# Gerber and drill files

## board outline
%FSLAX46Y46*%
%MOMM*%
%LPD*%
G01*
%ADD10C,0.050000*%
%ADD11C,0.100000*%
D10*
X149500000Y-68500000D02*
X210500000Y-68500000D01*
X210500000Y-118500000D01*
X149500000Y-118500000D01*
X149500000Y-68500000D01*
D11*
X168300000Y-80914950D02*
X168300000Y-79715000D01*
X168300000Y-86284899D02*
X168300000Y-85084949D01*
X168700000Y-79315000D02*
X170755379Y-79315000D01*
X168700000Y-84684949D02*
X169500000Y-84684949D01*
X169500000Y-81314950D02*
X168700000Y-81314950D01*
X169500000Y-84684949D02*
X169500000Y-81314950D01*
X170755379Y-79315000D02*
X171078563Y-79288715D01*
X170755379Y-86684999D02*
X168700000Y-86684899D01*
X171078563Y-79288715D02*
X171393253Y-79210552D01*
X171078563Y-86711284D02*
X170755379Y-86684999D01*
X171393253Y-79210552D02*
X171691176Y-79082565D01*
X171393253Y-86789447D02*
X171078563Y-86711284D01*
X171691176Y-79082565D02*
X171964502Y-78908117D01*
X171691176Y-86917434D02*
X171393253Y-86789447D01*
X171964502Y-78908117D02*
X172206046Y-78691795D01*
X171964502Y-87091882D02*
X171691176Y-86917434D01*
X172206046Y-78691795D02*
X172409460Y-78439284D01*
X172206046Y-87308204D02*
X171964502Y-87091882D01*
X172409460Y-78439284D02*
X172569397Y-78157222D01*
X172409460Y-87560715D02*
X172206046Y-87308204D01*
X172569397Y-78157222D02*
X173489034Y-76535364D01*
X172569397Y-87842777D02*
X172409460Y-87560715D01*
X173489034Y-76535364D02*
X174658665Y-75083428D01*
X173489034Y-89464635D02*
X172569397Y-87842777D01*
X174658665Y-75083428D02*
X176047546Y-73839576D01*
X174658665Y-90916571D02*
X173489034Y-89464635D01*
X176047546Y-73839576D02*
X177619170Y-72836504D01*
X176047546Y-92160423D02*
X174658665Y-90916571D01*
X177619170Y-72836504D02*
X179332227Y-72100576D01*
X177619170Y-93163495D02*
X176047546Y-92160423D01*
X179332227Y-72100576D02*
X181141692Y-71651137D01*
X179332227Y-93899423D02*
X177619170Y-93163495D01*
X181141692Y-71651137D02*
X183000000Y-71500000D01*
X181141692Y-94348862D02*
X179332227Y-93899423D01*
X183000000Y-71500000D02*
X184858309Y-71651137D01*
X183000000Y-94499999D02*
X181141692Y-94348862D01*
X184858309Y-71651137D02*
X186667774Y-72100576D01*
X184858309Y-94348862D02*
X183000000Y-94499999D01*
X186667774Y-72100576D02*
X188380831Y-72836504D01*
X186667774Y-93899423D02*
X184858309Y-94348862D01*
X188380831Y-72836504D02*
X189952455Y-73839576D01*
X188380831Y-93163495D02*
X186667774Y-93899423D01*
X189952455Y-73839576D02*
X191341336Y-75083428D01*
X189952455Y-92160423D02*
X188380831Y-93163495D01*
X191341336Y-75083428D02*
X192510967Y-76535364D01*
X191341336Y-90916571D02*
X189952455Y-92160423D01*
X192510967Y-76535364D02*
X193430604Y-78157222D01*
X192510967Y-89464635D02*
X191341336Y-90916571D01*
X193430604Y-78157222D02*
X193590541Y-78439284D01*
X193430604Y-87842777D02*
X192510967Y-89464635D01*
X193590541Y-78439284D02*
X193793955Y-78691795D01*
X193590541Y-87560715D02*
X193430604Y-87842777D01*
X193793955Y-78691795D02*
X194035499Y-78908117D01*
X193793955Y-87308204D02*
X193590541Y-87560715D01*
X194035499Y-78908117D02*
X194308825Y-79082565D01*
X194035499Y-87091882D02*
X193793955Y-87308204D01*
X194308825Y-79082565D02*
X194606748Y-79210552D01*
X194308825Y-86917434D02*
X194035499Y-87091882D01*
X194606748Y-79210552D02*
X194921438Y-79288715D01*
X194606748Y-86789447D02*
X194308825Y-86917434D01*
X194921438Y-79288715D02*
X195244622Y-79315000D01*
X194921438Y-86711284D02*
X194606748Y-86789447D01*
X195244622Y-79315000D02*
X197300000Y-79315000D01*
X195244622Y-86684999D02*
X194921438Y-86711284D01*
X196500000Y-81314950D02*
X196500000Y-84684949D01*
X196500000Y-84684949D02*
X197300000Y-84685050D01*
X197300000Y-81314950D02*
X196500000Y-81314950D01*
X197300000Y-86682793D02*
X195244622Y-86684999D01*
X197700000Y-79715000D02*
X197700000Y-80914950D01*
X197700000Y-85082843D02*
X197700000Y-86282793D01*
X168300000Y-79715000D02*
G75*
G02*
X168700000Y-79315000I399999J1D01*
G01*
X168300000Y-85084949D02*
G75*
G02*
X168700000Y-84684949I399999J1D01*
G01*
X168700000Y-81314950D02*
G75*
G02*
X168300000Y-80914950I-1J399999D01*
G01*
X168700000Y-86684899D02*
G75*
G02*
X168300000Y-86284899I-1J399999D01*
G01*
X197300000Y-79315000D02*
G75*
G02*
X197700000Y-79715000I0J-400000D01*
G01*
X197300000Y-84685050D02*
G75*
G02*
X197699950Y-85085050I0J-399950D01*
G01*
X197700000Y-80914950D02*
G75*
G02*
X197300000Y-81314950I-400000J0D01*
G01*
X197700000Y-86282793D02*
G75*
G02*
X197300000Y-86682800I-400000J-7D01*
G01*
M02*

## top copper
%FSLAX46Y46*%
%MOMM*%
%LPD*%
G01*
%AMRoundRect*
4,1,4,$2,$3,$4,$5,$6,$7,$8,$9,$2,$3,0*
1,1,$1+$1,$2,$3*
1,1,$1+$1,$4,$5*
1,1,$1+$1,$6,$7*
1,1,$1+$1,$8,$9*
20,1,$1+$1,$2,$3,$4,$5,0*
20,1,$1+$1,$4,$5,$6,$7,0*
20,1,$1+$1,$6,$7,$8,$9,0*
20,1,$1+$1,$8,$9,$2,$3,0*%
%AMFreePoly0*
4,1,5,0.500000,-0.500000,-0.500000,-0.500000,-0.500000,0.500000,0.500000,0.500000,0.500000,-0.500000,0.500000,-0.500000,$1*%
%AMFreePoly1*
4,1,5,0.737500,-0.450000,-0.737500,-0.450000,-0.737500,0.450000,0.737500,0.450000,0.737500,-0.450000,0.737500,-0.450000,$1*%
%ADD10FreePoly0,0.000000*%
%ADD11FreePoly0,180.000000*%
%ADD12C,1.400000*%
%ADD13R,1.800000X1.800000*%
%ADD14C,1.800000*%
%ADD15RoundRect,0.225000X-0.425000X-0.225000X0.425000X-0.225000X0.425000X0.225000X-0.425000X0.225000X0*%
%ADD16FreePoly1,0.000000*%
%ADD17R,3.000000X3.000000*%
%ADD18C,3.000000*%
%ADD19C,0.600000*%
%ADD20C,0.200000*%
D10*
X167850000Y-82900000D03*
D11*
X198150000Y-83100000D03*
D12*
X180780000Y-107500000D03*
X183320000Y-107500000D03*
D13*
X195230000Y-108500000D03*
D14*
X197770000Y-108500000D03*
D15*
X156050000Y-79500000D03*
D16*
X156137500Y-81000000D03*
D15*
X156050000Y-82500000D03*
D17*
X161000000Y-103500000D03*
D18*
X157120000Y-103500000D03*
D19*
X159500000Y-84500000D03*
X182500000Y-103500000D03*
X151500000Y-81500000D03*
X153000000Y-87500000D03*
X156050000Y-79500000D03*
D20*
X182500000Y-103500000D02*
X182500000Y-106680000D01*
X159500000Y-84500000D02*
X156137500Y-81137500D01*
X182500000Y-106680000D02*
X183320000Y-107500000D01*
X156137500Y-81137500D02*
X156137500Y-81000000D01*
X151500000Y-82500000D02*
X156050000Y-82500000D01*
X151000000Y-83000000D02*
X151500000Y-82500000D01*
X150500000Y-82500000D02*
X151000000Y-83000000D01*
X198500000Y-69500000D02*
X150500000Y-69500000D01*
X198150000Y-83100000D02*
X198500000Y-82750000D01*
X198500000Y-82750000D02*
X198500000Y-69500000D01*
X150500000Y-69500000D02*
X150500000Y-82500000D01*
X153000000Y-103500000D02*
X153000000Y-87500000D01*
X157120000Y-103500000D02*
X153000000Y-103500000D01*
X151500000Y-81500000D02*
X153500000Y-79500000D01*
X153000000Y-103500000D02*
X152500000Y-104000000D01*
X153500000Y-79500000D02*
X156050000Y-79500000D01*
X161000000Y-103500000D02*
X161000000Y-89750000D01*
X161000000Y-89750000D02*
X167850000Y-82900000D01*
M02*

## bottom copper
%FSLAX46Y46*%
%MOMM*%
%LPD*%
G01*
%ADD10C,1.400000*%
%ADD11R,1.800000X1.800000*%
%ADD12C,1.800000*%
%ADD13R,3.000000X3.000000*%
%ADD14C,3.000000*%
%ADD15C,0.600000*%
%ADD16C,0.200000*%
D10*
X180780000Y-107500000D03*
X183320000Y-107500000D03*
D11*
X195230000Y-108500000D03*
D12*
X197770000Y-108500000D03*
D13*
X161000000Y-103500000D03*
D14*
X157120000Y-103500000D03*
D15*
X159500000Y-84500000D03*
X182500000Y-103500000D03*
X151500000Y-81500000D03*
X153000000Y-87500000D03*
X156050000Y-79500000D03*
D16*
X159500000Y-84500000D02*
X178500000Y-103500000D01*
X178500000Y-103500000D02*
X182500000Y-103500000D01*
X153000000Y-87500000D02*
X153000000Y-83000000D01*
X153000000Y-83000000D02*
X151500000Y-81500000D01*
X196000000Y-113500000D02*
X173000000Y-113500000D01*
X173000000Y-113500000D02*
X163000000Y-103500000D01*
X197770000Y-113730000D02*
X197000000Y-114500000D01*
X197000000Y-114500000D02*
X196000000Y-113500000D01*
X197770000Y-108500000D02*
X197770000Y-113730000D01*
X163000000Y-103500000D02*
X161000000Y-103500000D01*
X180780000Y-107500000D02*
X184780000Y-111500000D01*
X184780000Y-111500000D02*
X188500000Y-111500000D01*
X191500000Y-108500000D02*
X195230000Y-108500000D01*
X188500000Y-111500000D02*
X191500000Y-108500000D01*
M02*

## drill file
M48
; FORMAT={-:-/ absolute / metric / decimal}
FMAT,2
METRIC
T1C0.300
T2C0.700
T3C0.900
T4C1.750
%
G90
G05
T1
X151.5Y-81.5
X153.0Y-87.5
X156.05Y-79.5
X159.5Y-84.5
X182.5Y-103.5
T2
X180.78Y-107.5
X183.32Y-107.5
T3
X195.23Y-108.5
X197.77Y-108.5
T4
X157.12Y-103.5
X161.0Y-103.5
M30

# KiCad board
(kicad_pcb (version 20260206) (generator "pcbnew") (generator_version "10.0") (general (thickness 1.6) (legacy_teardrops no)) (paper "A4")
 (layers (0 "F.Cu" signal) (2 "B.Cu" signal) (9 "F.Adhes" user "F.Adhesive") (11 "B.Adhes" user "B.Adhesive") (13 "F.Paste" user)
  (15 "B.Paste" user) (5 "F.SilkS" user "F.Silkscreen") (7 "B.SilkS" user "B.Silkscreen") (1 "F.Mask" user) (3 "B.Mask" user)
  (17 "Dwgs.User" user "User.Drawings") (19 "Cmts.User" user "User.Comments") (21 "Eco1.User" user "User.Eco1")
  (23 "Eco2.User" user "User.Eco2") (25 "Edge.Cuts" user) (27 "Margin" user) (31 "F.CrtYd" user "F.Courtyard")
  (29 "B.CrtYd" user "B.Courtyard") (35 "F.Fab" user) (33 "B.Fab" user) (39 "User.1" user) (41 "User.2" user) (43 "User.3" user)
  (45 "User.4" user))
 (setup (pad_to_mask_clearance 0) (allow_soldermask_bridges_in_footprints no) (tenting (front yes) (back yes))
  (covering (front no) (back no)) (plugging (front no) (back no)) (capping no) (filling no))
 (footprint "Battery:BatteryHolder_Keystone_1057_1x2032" (layer "F.Cu") (at 183 83)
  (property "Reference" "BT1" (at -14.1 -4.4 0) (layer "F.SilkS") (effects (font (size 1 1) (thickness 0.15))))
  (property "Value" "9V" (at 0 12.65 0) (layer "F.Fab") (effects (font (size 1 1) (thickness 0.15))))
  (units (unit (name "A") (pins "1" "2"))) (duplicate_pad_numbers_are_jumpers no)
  (fp_line (start -14.7 -2.08505) (end -14.7 -3.285) (stroke (width 0.1) (type solid)) (layer "Edge.Cuts"))
  (fp_line (start -14.7 3.284899) (end -14.7 2.084949) (stroke (width 0.1) (type solid)) (layer "Edge.Cuts"))
  (fp_line (start -14.3 -3.685) (end -12.244621 -3.685) (stroke (width 0.1) (type solid)) (layer "Edge.Cuts"))
  (fp_line (start -14.3 1.684949) (end -13.5 1.684949) (stroke (width 0.1) (type solid)) (layer "Edge.Cuts"))
  (fp_line (start -13.5 -1.68505) (end -14.3 -1.68505) (stroke (width 0.1) (type solid)) (layer "Edge.Cuts"))
  (fp_line (start -13.5 1.684949) (end -13.5 -1.68505) (stroke (width 0.1) (type solid)) (layer "Edge.Cuts"))
  (fp_line (start -12.244621 -3.685) (end -11.921437 -3.711285) (stroke (width 0.1) (type solid)) (layer "Edge.Cuts"))
  (fp_line (start -12.244621 3.684999) (end -14.3 3.684899) (stroke (width 0.1) (type solid)) (layer "Edge.Cuts"))
  (fp_line (start -11.921437 -3.711285) (end -11.606747 -3.789448) (stroke (width 0.1) (type solid)) (layer "Edge.Cuts"))
  (fp_line (start -11.921437 3.711284) (end -12.244621 3.684999) (stroke (width 0.1) (type solid)) (layer "Edge.Cuts"))
  (fp_line (start -11.606747 -3.789448) (end -11.308824 -3.917435) (stroke (width 0.1) (type solid)) (layer "Edge.Cuts"))
  (fp_line (start -11.606747 3.789447) (end -11.921437 3.711284) (stroke (width 0.1) (type solid)) (layer "Edge.Cuts"))
  (fp_line (start -11.308824 -3.917435) (end -11.035498 -4.091883) (stroke (width 0.1) (type solid)) (layer "Edge.Cuts"))
  (fp_line (start -11.308824 3.917434) (end -11.606747 3.789447) (stroke (width 0.1) (type solid)) (layer "Edge.Cuts"))
  (fp_line (start -11.035498 -4.091883) (end -10.793954 -4.308205) (stroke (width 0.1) (type solid)) (layer "Edge.Cuts"))
  (fp_line (start -11.035498 4.091882) (end -11.308824 3.917434) (stroke (width 0.1) (type solid)) (layer "Edge.Cuts"))
  (fp_line (start -10.793954 -4.308205) (end -10.59054 -4.560716) (stroke (width 0.1) (type solid)) (layer "Edge.Cuts"))
  (fp_line (start -10.793954 4.308204) (end -11.035498 4.091882) (stroke (width 0.1) (type solid)) (layer "Edge.Cuts"))
  (fp_line (start -10.59054 -4.560716) (end -10.430603 -4.842778) (stroke (width 0.1) (type solid)) (layer "Edge.Cuts"))
  (fp_line (start -10.59054 4.560715) (end -10.793954 4.308204) (stroke (width 0.1) (type solid)) (layer "Edge.Cuts"))
  (fp_line (start -10.430603 -4.842778) (end -9.510966 -6.464636) (stroke (width 0.1) (type solid)) (layer "Edge.Cuts"))
  (fp_line (start -10.430603 4.842777) (end -10.59054 4.560715) (stroke (width 0.1) (type solid)) (layer "Edge.Cuts"))
  (fp_line (start -9.510966 -6.464636) (end -8.341335 -7.916572) (stroke (width 0.1) (type solid)) (layer "Edge.Cuts"))
  (fp_line (start -9.510966 6.464635) (end -10.430603 4.842777) (stroke (width 0.1) (type solid)) (layer "Edge.Cuts"))
  (fp_line (start -8.341335 -7.916572) (end -6.952454 -9.160424) (stroke (width 0.1) (type solid)) (layer "Edge.Cuts"))
  (fp_line (start -8.341335 7.916571) (end -9.510966 6.464635) (stroke (width 0.1) (type solid)) (layer "Edge.Cuts"))
  (fp_line (start -6.952454 -9.160424) (end -5.38083 -10.163496) (stroke (width 0.1) (type solid)) (layer "Edge.Cuts"))
  (fp_line (start -6.952454 9.160423) (end -8.341335 7.916571) (stroke (width 0.1) (type solid)) (layer "Edge.Cuts"))
  (fp_line (start -5.38083 -10.163496) (end -3.667773 -10.899424) (stroke (width 0.1) (type solid)) (layer "Edge.Cuts"))
  (fp_line (start -5.38083 10.163495) (end -6.952454 9.160423) (stroke (width 0.1) (type solid)) (layer "Edge.Cuts"))
  (fp_line (start -3.667773 -10.899424) (end -1.858308 -11.348863) (stroke (width 0.1) (type solid)) (layer "Edge.Cuts"))
  (fp_line (start -3.667773 10.899423) (end -5.38083 10.163495) (stroke (width 0.1) (type solid)) (layer "Edge.Cuts"))
  (fp_line (start -1.858308 -11.348863) (end 0 -11.5) (stroke (width 0.1) (type solid)) (layer "Edge.Cuts"))
  (fp_line (start -1.858308 11.348862) (end -3.667773 10.899423) (stroke (width 0.1) (type solid)) (layer "Edge.Cuts"))
  (fp_line (start 0 -11.5) (end 1.858309 -11.348863) (stroke (width 0.1) (type solid)) (layer "Edge.Cuts"))
  (fp_line (start 0 11.499999) (end -1.858308 11.348862) (stroke (width 0.1) (type solid)) (layer "Edge.Cuts"))
  (fp_line (start 1.858309 -11.348863) (end 3.667774 -10.899424) (stroke (width 0.1) (type solid)) (layer "Edge.Cuts"))
  (fp_line (start 1.858309 11.348862) (end 0 11.499999) (stroke (width 0.1) (type solid)) (layer "Edge.Cuts"))
  (fp_line (start 3.667774 -10.899424) (end 5.380831 -10.163496) (stroke (width 0.1) (type solid)) (layer "Edge.Cuts"))
  (fp_line (start 3.667774 10.899423) (end 1.858309 11.348862) (stroke (width 0.1) (type solid)) (layer "Edge.Cuts"))
  (fp_line (start 5.380831 -10.163496) (end 6.952455 -9.160424) (stroke (width 0.1) (type solid)) (layer "Edge.Cuts"))
  (fp_line (start 5.380831 10.163495) (end 3.667774 10.899423) (stroke (width 0.1) (type solid)) (layer "Edge.Cuts"))
  (fp_line (start 6.952455 -9.160424) (end 8.341336 -7.916572) (stroke (width 0.1) (type solid)) (layer "Edge.Cuts"))
  (fp_line (start 6.952455 9.160423) (end 5.380831 10.163495) (stroke (width 0.1) (type solid)) (layer "Edge.Cuts"))
  (fp_line (start 8.341336 -7.916572) (end 9.510967 -6.464636) (stroke (width 0.1) (type solid)) (layer "Edge.Cuts"))
  (fp_line (start 8.341336 7.916571) (end 6.952455 9.160423) (stroke (width 0.1) (type solid)) (layer "Edge.Cuts"))
  (fp_line (start 9.510967 -6.464636) (end 10.430604 -4.842778) (stroke (width 0.1) (type solid)) (layer "Edge.Cuts"))
  (fp_line (start 9.510967 6.464635) (end 8.341336 7.916571) (stroke (width 0.1) (type solid)) (layer "Edge.Cuts"))
  (fp_line (start 10.430604 -4.842778) (end 10.590541 -4.560716) (stroke (width 0.1) (type solid)) (layer "Edge.Cuts"))
  (fp_line (start 10.430604 4.842777) (end 9.510967 6.464635) (stroke (width 0.1) (type solid)) (layer "Edge.Cuts"))
  (fp_line (start 10.590541 -4.560716) (end 10.793955 -4.308205) (stroke (width 0.1) (type solid)) (layer "Edge.Cuts"))
  (fp_line (start 10.590541 4.560715) (end 10.430604 4.842777) (stroke (width 0.1) (type solid)) (layer "Edge.Cuts"))
  (fp_line (start 10.793955 -4.308205) (end 11.035499 -4.091883) (stroke (width 0.1) (type solid)) (layer "Edge.Cuts"))
  (fp_line (start 10.793955 4.308204) (end 10.590541 4.560715) (stroke (width 0.1) (type solid)) (layer "Edge.Cuts"))
  (fp_line (start 11.035499 -4.091883) (end 11.308825 -3.917435) (stroke (width 0.1) (type solid)) (layer "Edge.Cuts"))
  (fp_line (start 11.035499 4.091882) (end 10.793955 4.308204) (stroke (width 0.1) (type solid)) (layer "Edge.Cuts"))
  (fp_line (start 11.308825 -3.917435) (end 11.606748 -3.789448) (stroke (width 0.1) (type solid)) (layer "Edge.Cuts"))
  (fp_line (start 11.308825 3.917434) (end 11.035499 4.091882) (stroke (width 0.1) (type solid)) (layer "Edge.Cuts"))
  (fp_line (start 11.606748 -3.789448) (end 11.921438 -3.711285) (stroke (width 0.1) (type solid)) (layer "Edge.Cuts"))
  (fp_line (start 11.606748 3.789447) (end 11.308825 3.917434) (stroke (width 0.1) (type solid)) (layer "Edge.Cuts"))
  (fp_line (start 11.921438 -3.711285) (end 12.244622 -3.685) (stroke (width 0.1) (type solid)) (layer "Edge.Cuts"))
  (fp_line (start 11.921438 3.711284) (end 11.606748 3.789447) (stroke (width 0.1) (type solid)) (layer "Edge.Cuts"))
  (fp_line (start 12.244622 -3.685) (end 14.3 -3.685) (stroke (width 0.1) (type solid)) (layer "Edge.Cuts"))
  (fp_line (start 12.244622 3.684999) (end 11.921438 3.711284) (stroke (width 0.1) (type solid)) (layer "Edge.Cuts"))
  (fp_line (start 13.5 -1.68505) (end 13.5 1.684949) (stroke (width 0.1) (type solid)) (layer "Edge.Cuts"))
  (fp_line (start 13.5 1.684949) (end 14.3 1.68505) (stroke (width 0.1) (type solid)) (layer "Edge.Cuts"))
  (fp_line (start 14.3 -1.68505) (end 13.5 -1.68505) (stroke (width 0.1) (type solid)) (layer "Edge.Cuts"))
  (fp_line (start 14.3 3.682793) (end 12.244622 3.684999) (stroke (width 0.1) (type solid)) (layer "Edge.Cuts"))
  (fp_line (start 14.7 -3.285) (end 14.7 -2.08505) (stroke (width 0.1) (type solid)) (layer "Edge.Cuts"))
  (fp_line (start 14.7 2.082843) (end 14.7 3.282793) (stroke (width 0.1) (type solid)) (layer "Edge.Cuts"))
  (fp_arc (start -14.7 -3.285) (mid -14.582843 -3.567843) (end -14.3 -3.685) (stroke (width 0.1) (type solid)) (layer "Edge.Cuts"))
  (fp_arc (start -14.7 2.084949) (mid -14.582843 1.802106) (end -14.3 1.684949) (stroke (width 0.1) (type solid)) (layer "Edge.Cuts"))
  (fp_arc (start -14.3 -1.68505) (mid -14.582843 -1.802207) (end -14.7 -2.08505) (stroke (width 0.1) (type solid)) (layer "Edge.Cuts"))
  (fp_arc (start -14.3 3.684899) (mid -14.582843 3.567742) (end -14.7 3.284899) (stroke (width 0.1) (type solid)) (layer "Edge.Cuts"))
  (fp_arc (start 14.3 -3.685) (mid 14.582843 -3.567843) (end 14.7 -3.285) (stroke (width 0.1) (type solid)) (layer "Edge.Cuts"))
  (fp_arc (start 14.3 1.68505) (mid 14.582843 1.802207) (end 14.7 2.08505) (stroke (width 0.1) (type solid)) (layer "Edge.Cuts"))
  (fp_arc (start 14.7 -2.08505) (mid 14.582843 -1.802207) (end 14.3 -1.68505) (stroke (width 0.1) (type solid)) (layer "Edge.Cuts"))
  (fp_arc (start 14.7 3.282793) (mid 14.582843 3.565636) (end 14.3 3.682793) (stroke (width 0.1) (type solid)) (layer "Edge.Cuts"))
  (pad "1" smd custom (at -15.15 -0.1) (size 1 1) (layers "F.Cu" "F.Mask" "F.Paste") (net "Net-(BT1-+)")
   (options (clearance outline) (anchor rect)) (primitives))
  (pad "2" smd custom (at 15.15 0.1 180) (size 1 1) (layers "F.Cu" "F.Mask" "F.Paste") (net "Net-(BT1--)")
   (options (clearance outline) (anchor rect)) (primitives)))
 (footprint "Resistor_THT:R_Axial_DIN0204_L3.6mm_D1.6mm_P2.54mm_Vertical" (layer "F.Cu") (at 180.78 107.5)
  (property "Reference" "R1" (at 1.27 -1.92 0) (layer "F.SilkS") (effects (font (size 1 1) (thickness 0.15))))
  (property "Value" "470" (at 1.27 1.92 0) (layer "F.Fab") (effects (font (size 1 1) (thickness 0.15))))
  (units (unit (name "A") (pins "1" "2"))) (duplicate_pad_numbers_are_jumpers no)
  (pad "1" thru_hole circle (at 0 0) (size 1.4 1.4) (drill 0.7) (layers "*.Cu" "*.Mask") (remove_unused_layers no) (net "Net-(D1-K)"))
  (pad "2" thru_hole circle (at 2.54 0) (size 1.4 1.4) (drill 0.7) (layers "*.Cu" "*.Mask") (remove_unused_layers no) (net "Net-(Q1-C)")))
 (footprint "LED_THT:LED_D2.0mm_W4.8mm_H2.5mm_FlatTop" (layer "F.Cu") (at 195.23 108.5)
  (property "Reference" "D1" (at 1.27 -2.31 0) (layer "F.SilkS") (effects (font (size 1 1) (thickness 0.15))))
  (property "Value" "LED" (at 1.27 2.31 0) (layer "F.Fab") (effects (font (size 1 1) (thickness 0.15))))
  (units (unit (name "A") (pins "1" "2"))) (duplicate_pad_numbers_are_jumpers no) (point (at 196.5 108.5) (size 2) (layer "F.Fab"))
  (pad "1" thru_hole rect (at 0 0) (size 1.8 1.8) (drill 0.9) (layers "*.Cu" "*.Mask") (remove_unused_layers no) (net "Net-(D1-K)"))
  (pad "2" thru_hole circle (at 2.54 0) (size 1.8 1.8) (drill 0.9) (layers "*.Cu" "*.Mask") (remove_unused_layers no) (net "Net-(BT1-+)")))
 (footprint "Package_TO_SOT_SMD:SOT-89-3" (layer "F.Cu") (at 158 81)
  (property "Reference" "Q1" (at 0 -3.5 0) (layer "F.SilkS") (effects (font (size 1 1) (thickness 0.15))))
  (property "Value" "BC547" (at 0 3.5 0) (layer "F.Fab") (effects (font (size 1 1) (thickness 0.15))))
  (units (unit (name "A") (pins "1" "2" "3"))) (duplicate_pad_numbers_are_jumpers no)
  (pad "1" smd roundrect (at -1.95 -1.5) (size 1.3 0.9) (layers "F.Cu" "F.Mask" "F.Paste") (roundrect_rratio 0.25) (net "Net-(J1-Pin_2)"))
  (pad "2" smd custom (at -1.8625 0) (size 1.475 0.9) (layers "F.Cu" "F.Mask" "F.Paste") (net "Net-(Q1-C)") (zone_connect 2)
   (thermal_bridge_angle 45) (options (clearance outline) (anchor rect)) (primitives))
  (pad "3" smd roundrect (at -1.95 1.5) (size 1.3 0.9) (layers "F.Cu" "F.Mask" "F.Paste") (roundrect_rratio 0.25) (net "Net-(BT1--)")))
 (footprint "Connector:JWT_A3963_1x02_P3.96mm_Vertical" (layer "B.Cu") (at 161 103.5 180)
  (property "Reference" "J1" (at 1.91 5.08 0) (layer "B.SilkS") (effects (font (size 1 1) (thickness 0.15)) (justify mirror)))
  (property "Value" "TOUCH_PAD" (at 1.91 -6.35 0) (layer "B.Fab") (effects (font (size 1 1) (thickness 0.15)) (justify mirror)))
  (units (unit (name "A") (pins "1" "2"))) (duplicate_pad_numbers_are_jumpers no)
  (pad "1" thru_hole rect (at 0 0 180) (size 3 3) (drill 1.75) (layers "*.Cu" "*.Mask") (remove_unused_layers no) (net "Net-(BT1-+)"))
  (pad "2" thru_hole circle (at 3.88 0 180) (size 3 3) (drill 1.75) (layers "*.Cu" "*.Mask") (remove_unused_layers no)
   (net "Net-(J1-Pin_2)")))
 (gr_rect (start 149.5 68.5) (end 210.5 118.5) (stroke (width 0.05) (type default)) (fill no) (layer "Edge.Cuts"))
 (segment (start 182.5 103.5) (end 182.5 106.68) (width 0.2) (layer "F.Cu") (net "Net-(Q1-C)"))
 (segment (start 159.5 84.5) (end 156.1375 81.1375) (width 0.2) (layer "F.Cu") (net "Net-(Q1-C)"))
 (segment (start 182.5 106.68) (end 183.32 107.5) (width 0.2) (layer "F.Cu") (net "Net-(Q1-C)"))
 (segment (start 156.1375 81.1375) (end 156.1375 81) (width 0.2) (layer "F.Cu") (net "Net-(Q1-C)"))
 (via (at 159.5 84.5) (size 0.6) (drill 0.3) (layers "F.Cu" "B.Cu") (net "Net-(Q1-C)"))
 (via (at 182.5 103.5) (size 0.6) (drill 0.3) (layers "F.Cu" "B.Cu") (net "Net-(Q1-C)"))
 (segment (start 159.5 84.5) (end 178.5 103.5) (width 0.2) (layer "B.Cu") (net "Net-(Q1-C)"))
 (segment (start 178.5 103.5) (end 182.5 103.5) (width 0.2) (layer "B.Cu") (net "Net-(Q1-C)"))
 (segment (start 151.5 82.5) (end 156.05 82.5) (width 0.2) (layer "F.Cu") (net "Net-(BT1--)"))
 (segment (start 151 83) (end 151.5 82.5) (width 0.2) (layer "F.Cu") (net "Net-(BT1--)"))
 (segment (start 150.5 82.5) (end 151 83) (width 0.2) (layer "F.Cu") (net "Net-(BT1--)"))
 (segment (start 198.5 69.5) (end 150.5 69.5) (width 0.2) (layer "F.Cu") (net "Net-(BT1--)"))
 (segment (start 198.15 83.1) (end 198.5 82.75) (width 0.2) (layer "F.Cu") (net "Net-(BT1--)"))
 (segment (start 198.5 82.75) (end 198.5 69.5) (width 0.2) (layer "F.Cu") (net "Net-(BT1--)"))
 (segment (start 150.5 69.5) (end 150.5 82.5) (width 0.2) (layer "F.Cu") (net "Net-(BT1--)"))
 (segment (start 153 103.5) (end 153 87.5) (width 0.2) (layer "F.Cu") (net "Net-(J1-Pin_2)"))
 (segment (start 157.12 103.5) (end 153 103.5) (width 0.2) (layer "F.Cu") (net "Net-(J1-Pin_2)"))
 (segment (start 151.5 81.5) (end 153.5 79.5) (width 0.2) (layer "F.Cu") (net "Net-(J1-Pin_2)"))
 (segment (start 153 103.5) (end 152.5 104) (width 0.2) (layer "F.Cu") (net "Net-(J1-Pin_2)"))
 (segment (start 153.5 79.5) (end 156.05 79.5) (width 0.2) (layer "F.Cu") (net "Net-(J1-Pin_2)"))
 (via (at 151.5 81.5) (size 0.6) (drill 0.3) (layers "F.Cu" "B.Cu") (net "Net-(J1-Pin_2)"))
 (via (at 153 87.5) (size 0.6) (drill 0.3) (layers "F.Cu" "B.Cu") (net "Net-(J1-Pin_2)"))
 (via (at 156.05 79.5) (size 0.6) (drill 0.3) (layers "F.Cu" "B.Cu") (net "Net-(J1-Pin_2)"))
 (segment (start 153 87.5) (end 153 83) (width 0.2) (layer "B.Cu") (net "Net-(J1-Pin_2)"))
 (segment (start 153 83) (end 151.5 81.5) (width 0.2) (layer "B.Cu") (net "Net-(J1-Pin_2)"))
 (segment (start 161 103.5) (end 161 89.75) (width 0.2) (layer "F.Cu") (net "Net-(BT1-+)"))
 (segment (start 161 89.75) (end 167.85 82.9) (width 0.2) (layer "F.Cu") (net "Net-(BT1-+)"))
 (segment (start 196 113.5) (end 173 113.5) (width 0.2) (layer "B.Cu") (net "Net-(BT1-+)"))
 (segment (start 173 113.5) (end 163 103.5) (width 0.2) (layer "B.Cu") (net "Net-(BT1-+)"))
 (segment (start 197.77 113.73) (end 197 114.5) (width 0.2) (layer "B.Cu") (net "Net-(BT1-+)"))
 (segment (start 197 114.5) (end 196 113.5) (width 0.2) (layer "B.Cu") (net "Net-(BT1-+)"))
 (segment (start 197.77 108.5) (end 197.77 113.73) (width 0.2) (layer "B.Cu") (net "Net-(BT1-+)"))
 (segment (start 163 103.5) (end 161 103.5) (width 0.2) (layer "B.Cu") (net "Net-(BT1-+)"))
 (segment (start 180.78 107.5) (end 184.78 111.5) (width 0.2) (layer "B.Cu") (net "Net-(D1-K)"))
 (segment (start 184.78 111.5) (end 188.5 111.5) (width 0.2) (layer "B.Cu") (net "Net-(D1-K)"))
 (segment (start 191.5 108.5) (end 195.23 108.5) (width 0.2) (layer "B.Cu") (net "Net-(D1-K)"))
 (segment (start 188.5 111.5) (end 191.5 108.5) (width 0.2) (layer "B.Cu") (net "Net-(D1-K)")))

